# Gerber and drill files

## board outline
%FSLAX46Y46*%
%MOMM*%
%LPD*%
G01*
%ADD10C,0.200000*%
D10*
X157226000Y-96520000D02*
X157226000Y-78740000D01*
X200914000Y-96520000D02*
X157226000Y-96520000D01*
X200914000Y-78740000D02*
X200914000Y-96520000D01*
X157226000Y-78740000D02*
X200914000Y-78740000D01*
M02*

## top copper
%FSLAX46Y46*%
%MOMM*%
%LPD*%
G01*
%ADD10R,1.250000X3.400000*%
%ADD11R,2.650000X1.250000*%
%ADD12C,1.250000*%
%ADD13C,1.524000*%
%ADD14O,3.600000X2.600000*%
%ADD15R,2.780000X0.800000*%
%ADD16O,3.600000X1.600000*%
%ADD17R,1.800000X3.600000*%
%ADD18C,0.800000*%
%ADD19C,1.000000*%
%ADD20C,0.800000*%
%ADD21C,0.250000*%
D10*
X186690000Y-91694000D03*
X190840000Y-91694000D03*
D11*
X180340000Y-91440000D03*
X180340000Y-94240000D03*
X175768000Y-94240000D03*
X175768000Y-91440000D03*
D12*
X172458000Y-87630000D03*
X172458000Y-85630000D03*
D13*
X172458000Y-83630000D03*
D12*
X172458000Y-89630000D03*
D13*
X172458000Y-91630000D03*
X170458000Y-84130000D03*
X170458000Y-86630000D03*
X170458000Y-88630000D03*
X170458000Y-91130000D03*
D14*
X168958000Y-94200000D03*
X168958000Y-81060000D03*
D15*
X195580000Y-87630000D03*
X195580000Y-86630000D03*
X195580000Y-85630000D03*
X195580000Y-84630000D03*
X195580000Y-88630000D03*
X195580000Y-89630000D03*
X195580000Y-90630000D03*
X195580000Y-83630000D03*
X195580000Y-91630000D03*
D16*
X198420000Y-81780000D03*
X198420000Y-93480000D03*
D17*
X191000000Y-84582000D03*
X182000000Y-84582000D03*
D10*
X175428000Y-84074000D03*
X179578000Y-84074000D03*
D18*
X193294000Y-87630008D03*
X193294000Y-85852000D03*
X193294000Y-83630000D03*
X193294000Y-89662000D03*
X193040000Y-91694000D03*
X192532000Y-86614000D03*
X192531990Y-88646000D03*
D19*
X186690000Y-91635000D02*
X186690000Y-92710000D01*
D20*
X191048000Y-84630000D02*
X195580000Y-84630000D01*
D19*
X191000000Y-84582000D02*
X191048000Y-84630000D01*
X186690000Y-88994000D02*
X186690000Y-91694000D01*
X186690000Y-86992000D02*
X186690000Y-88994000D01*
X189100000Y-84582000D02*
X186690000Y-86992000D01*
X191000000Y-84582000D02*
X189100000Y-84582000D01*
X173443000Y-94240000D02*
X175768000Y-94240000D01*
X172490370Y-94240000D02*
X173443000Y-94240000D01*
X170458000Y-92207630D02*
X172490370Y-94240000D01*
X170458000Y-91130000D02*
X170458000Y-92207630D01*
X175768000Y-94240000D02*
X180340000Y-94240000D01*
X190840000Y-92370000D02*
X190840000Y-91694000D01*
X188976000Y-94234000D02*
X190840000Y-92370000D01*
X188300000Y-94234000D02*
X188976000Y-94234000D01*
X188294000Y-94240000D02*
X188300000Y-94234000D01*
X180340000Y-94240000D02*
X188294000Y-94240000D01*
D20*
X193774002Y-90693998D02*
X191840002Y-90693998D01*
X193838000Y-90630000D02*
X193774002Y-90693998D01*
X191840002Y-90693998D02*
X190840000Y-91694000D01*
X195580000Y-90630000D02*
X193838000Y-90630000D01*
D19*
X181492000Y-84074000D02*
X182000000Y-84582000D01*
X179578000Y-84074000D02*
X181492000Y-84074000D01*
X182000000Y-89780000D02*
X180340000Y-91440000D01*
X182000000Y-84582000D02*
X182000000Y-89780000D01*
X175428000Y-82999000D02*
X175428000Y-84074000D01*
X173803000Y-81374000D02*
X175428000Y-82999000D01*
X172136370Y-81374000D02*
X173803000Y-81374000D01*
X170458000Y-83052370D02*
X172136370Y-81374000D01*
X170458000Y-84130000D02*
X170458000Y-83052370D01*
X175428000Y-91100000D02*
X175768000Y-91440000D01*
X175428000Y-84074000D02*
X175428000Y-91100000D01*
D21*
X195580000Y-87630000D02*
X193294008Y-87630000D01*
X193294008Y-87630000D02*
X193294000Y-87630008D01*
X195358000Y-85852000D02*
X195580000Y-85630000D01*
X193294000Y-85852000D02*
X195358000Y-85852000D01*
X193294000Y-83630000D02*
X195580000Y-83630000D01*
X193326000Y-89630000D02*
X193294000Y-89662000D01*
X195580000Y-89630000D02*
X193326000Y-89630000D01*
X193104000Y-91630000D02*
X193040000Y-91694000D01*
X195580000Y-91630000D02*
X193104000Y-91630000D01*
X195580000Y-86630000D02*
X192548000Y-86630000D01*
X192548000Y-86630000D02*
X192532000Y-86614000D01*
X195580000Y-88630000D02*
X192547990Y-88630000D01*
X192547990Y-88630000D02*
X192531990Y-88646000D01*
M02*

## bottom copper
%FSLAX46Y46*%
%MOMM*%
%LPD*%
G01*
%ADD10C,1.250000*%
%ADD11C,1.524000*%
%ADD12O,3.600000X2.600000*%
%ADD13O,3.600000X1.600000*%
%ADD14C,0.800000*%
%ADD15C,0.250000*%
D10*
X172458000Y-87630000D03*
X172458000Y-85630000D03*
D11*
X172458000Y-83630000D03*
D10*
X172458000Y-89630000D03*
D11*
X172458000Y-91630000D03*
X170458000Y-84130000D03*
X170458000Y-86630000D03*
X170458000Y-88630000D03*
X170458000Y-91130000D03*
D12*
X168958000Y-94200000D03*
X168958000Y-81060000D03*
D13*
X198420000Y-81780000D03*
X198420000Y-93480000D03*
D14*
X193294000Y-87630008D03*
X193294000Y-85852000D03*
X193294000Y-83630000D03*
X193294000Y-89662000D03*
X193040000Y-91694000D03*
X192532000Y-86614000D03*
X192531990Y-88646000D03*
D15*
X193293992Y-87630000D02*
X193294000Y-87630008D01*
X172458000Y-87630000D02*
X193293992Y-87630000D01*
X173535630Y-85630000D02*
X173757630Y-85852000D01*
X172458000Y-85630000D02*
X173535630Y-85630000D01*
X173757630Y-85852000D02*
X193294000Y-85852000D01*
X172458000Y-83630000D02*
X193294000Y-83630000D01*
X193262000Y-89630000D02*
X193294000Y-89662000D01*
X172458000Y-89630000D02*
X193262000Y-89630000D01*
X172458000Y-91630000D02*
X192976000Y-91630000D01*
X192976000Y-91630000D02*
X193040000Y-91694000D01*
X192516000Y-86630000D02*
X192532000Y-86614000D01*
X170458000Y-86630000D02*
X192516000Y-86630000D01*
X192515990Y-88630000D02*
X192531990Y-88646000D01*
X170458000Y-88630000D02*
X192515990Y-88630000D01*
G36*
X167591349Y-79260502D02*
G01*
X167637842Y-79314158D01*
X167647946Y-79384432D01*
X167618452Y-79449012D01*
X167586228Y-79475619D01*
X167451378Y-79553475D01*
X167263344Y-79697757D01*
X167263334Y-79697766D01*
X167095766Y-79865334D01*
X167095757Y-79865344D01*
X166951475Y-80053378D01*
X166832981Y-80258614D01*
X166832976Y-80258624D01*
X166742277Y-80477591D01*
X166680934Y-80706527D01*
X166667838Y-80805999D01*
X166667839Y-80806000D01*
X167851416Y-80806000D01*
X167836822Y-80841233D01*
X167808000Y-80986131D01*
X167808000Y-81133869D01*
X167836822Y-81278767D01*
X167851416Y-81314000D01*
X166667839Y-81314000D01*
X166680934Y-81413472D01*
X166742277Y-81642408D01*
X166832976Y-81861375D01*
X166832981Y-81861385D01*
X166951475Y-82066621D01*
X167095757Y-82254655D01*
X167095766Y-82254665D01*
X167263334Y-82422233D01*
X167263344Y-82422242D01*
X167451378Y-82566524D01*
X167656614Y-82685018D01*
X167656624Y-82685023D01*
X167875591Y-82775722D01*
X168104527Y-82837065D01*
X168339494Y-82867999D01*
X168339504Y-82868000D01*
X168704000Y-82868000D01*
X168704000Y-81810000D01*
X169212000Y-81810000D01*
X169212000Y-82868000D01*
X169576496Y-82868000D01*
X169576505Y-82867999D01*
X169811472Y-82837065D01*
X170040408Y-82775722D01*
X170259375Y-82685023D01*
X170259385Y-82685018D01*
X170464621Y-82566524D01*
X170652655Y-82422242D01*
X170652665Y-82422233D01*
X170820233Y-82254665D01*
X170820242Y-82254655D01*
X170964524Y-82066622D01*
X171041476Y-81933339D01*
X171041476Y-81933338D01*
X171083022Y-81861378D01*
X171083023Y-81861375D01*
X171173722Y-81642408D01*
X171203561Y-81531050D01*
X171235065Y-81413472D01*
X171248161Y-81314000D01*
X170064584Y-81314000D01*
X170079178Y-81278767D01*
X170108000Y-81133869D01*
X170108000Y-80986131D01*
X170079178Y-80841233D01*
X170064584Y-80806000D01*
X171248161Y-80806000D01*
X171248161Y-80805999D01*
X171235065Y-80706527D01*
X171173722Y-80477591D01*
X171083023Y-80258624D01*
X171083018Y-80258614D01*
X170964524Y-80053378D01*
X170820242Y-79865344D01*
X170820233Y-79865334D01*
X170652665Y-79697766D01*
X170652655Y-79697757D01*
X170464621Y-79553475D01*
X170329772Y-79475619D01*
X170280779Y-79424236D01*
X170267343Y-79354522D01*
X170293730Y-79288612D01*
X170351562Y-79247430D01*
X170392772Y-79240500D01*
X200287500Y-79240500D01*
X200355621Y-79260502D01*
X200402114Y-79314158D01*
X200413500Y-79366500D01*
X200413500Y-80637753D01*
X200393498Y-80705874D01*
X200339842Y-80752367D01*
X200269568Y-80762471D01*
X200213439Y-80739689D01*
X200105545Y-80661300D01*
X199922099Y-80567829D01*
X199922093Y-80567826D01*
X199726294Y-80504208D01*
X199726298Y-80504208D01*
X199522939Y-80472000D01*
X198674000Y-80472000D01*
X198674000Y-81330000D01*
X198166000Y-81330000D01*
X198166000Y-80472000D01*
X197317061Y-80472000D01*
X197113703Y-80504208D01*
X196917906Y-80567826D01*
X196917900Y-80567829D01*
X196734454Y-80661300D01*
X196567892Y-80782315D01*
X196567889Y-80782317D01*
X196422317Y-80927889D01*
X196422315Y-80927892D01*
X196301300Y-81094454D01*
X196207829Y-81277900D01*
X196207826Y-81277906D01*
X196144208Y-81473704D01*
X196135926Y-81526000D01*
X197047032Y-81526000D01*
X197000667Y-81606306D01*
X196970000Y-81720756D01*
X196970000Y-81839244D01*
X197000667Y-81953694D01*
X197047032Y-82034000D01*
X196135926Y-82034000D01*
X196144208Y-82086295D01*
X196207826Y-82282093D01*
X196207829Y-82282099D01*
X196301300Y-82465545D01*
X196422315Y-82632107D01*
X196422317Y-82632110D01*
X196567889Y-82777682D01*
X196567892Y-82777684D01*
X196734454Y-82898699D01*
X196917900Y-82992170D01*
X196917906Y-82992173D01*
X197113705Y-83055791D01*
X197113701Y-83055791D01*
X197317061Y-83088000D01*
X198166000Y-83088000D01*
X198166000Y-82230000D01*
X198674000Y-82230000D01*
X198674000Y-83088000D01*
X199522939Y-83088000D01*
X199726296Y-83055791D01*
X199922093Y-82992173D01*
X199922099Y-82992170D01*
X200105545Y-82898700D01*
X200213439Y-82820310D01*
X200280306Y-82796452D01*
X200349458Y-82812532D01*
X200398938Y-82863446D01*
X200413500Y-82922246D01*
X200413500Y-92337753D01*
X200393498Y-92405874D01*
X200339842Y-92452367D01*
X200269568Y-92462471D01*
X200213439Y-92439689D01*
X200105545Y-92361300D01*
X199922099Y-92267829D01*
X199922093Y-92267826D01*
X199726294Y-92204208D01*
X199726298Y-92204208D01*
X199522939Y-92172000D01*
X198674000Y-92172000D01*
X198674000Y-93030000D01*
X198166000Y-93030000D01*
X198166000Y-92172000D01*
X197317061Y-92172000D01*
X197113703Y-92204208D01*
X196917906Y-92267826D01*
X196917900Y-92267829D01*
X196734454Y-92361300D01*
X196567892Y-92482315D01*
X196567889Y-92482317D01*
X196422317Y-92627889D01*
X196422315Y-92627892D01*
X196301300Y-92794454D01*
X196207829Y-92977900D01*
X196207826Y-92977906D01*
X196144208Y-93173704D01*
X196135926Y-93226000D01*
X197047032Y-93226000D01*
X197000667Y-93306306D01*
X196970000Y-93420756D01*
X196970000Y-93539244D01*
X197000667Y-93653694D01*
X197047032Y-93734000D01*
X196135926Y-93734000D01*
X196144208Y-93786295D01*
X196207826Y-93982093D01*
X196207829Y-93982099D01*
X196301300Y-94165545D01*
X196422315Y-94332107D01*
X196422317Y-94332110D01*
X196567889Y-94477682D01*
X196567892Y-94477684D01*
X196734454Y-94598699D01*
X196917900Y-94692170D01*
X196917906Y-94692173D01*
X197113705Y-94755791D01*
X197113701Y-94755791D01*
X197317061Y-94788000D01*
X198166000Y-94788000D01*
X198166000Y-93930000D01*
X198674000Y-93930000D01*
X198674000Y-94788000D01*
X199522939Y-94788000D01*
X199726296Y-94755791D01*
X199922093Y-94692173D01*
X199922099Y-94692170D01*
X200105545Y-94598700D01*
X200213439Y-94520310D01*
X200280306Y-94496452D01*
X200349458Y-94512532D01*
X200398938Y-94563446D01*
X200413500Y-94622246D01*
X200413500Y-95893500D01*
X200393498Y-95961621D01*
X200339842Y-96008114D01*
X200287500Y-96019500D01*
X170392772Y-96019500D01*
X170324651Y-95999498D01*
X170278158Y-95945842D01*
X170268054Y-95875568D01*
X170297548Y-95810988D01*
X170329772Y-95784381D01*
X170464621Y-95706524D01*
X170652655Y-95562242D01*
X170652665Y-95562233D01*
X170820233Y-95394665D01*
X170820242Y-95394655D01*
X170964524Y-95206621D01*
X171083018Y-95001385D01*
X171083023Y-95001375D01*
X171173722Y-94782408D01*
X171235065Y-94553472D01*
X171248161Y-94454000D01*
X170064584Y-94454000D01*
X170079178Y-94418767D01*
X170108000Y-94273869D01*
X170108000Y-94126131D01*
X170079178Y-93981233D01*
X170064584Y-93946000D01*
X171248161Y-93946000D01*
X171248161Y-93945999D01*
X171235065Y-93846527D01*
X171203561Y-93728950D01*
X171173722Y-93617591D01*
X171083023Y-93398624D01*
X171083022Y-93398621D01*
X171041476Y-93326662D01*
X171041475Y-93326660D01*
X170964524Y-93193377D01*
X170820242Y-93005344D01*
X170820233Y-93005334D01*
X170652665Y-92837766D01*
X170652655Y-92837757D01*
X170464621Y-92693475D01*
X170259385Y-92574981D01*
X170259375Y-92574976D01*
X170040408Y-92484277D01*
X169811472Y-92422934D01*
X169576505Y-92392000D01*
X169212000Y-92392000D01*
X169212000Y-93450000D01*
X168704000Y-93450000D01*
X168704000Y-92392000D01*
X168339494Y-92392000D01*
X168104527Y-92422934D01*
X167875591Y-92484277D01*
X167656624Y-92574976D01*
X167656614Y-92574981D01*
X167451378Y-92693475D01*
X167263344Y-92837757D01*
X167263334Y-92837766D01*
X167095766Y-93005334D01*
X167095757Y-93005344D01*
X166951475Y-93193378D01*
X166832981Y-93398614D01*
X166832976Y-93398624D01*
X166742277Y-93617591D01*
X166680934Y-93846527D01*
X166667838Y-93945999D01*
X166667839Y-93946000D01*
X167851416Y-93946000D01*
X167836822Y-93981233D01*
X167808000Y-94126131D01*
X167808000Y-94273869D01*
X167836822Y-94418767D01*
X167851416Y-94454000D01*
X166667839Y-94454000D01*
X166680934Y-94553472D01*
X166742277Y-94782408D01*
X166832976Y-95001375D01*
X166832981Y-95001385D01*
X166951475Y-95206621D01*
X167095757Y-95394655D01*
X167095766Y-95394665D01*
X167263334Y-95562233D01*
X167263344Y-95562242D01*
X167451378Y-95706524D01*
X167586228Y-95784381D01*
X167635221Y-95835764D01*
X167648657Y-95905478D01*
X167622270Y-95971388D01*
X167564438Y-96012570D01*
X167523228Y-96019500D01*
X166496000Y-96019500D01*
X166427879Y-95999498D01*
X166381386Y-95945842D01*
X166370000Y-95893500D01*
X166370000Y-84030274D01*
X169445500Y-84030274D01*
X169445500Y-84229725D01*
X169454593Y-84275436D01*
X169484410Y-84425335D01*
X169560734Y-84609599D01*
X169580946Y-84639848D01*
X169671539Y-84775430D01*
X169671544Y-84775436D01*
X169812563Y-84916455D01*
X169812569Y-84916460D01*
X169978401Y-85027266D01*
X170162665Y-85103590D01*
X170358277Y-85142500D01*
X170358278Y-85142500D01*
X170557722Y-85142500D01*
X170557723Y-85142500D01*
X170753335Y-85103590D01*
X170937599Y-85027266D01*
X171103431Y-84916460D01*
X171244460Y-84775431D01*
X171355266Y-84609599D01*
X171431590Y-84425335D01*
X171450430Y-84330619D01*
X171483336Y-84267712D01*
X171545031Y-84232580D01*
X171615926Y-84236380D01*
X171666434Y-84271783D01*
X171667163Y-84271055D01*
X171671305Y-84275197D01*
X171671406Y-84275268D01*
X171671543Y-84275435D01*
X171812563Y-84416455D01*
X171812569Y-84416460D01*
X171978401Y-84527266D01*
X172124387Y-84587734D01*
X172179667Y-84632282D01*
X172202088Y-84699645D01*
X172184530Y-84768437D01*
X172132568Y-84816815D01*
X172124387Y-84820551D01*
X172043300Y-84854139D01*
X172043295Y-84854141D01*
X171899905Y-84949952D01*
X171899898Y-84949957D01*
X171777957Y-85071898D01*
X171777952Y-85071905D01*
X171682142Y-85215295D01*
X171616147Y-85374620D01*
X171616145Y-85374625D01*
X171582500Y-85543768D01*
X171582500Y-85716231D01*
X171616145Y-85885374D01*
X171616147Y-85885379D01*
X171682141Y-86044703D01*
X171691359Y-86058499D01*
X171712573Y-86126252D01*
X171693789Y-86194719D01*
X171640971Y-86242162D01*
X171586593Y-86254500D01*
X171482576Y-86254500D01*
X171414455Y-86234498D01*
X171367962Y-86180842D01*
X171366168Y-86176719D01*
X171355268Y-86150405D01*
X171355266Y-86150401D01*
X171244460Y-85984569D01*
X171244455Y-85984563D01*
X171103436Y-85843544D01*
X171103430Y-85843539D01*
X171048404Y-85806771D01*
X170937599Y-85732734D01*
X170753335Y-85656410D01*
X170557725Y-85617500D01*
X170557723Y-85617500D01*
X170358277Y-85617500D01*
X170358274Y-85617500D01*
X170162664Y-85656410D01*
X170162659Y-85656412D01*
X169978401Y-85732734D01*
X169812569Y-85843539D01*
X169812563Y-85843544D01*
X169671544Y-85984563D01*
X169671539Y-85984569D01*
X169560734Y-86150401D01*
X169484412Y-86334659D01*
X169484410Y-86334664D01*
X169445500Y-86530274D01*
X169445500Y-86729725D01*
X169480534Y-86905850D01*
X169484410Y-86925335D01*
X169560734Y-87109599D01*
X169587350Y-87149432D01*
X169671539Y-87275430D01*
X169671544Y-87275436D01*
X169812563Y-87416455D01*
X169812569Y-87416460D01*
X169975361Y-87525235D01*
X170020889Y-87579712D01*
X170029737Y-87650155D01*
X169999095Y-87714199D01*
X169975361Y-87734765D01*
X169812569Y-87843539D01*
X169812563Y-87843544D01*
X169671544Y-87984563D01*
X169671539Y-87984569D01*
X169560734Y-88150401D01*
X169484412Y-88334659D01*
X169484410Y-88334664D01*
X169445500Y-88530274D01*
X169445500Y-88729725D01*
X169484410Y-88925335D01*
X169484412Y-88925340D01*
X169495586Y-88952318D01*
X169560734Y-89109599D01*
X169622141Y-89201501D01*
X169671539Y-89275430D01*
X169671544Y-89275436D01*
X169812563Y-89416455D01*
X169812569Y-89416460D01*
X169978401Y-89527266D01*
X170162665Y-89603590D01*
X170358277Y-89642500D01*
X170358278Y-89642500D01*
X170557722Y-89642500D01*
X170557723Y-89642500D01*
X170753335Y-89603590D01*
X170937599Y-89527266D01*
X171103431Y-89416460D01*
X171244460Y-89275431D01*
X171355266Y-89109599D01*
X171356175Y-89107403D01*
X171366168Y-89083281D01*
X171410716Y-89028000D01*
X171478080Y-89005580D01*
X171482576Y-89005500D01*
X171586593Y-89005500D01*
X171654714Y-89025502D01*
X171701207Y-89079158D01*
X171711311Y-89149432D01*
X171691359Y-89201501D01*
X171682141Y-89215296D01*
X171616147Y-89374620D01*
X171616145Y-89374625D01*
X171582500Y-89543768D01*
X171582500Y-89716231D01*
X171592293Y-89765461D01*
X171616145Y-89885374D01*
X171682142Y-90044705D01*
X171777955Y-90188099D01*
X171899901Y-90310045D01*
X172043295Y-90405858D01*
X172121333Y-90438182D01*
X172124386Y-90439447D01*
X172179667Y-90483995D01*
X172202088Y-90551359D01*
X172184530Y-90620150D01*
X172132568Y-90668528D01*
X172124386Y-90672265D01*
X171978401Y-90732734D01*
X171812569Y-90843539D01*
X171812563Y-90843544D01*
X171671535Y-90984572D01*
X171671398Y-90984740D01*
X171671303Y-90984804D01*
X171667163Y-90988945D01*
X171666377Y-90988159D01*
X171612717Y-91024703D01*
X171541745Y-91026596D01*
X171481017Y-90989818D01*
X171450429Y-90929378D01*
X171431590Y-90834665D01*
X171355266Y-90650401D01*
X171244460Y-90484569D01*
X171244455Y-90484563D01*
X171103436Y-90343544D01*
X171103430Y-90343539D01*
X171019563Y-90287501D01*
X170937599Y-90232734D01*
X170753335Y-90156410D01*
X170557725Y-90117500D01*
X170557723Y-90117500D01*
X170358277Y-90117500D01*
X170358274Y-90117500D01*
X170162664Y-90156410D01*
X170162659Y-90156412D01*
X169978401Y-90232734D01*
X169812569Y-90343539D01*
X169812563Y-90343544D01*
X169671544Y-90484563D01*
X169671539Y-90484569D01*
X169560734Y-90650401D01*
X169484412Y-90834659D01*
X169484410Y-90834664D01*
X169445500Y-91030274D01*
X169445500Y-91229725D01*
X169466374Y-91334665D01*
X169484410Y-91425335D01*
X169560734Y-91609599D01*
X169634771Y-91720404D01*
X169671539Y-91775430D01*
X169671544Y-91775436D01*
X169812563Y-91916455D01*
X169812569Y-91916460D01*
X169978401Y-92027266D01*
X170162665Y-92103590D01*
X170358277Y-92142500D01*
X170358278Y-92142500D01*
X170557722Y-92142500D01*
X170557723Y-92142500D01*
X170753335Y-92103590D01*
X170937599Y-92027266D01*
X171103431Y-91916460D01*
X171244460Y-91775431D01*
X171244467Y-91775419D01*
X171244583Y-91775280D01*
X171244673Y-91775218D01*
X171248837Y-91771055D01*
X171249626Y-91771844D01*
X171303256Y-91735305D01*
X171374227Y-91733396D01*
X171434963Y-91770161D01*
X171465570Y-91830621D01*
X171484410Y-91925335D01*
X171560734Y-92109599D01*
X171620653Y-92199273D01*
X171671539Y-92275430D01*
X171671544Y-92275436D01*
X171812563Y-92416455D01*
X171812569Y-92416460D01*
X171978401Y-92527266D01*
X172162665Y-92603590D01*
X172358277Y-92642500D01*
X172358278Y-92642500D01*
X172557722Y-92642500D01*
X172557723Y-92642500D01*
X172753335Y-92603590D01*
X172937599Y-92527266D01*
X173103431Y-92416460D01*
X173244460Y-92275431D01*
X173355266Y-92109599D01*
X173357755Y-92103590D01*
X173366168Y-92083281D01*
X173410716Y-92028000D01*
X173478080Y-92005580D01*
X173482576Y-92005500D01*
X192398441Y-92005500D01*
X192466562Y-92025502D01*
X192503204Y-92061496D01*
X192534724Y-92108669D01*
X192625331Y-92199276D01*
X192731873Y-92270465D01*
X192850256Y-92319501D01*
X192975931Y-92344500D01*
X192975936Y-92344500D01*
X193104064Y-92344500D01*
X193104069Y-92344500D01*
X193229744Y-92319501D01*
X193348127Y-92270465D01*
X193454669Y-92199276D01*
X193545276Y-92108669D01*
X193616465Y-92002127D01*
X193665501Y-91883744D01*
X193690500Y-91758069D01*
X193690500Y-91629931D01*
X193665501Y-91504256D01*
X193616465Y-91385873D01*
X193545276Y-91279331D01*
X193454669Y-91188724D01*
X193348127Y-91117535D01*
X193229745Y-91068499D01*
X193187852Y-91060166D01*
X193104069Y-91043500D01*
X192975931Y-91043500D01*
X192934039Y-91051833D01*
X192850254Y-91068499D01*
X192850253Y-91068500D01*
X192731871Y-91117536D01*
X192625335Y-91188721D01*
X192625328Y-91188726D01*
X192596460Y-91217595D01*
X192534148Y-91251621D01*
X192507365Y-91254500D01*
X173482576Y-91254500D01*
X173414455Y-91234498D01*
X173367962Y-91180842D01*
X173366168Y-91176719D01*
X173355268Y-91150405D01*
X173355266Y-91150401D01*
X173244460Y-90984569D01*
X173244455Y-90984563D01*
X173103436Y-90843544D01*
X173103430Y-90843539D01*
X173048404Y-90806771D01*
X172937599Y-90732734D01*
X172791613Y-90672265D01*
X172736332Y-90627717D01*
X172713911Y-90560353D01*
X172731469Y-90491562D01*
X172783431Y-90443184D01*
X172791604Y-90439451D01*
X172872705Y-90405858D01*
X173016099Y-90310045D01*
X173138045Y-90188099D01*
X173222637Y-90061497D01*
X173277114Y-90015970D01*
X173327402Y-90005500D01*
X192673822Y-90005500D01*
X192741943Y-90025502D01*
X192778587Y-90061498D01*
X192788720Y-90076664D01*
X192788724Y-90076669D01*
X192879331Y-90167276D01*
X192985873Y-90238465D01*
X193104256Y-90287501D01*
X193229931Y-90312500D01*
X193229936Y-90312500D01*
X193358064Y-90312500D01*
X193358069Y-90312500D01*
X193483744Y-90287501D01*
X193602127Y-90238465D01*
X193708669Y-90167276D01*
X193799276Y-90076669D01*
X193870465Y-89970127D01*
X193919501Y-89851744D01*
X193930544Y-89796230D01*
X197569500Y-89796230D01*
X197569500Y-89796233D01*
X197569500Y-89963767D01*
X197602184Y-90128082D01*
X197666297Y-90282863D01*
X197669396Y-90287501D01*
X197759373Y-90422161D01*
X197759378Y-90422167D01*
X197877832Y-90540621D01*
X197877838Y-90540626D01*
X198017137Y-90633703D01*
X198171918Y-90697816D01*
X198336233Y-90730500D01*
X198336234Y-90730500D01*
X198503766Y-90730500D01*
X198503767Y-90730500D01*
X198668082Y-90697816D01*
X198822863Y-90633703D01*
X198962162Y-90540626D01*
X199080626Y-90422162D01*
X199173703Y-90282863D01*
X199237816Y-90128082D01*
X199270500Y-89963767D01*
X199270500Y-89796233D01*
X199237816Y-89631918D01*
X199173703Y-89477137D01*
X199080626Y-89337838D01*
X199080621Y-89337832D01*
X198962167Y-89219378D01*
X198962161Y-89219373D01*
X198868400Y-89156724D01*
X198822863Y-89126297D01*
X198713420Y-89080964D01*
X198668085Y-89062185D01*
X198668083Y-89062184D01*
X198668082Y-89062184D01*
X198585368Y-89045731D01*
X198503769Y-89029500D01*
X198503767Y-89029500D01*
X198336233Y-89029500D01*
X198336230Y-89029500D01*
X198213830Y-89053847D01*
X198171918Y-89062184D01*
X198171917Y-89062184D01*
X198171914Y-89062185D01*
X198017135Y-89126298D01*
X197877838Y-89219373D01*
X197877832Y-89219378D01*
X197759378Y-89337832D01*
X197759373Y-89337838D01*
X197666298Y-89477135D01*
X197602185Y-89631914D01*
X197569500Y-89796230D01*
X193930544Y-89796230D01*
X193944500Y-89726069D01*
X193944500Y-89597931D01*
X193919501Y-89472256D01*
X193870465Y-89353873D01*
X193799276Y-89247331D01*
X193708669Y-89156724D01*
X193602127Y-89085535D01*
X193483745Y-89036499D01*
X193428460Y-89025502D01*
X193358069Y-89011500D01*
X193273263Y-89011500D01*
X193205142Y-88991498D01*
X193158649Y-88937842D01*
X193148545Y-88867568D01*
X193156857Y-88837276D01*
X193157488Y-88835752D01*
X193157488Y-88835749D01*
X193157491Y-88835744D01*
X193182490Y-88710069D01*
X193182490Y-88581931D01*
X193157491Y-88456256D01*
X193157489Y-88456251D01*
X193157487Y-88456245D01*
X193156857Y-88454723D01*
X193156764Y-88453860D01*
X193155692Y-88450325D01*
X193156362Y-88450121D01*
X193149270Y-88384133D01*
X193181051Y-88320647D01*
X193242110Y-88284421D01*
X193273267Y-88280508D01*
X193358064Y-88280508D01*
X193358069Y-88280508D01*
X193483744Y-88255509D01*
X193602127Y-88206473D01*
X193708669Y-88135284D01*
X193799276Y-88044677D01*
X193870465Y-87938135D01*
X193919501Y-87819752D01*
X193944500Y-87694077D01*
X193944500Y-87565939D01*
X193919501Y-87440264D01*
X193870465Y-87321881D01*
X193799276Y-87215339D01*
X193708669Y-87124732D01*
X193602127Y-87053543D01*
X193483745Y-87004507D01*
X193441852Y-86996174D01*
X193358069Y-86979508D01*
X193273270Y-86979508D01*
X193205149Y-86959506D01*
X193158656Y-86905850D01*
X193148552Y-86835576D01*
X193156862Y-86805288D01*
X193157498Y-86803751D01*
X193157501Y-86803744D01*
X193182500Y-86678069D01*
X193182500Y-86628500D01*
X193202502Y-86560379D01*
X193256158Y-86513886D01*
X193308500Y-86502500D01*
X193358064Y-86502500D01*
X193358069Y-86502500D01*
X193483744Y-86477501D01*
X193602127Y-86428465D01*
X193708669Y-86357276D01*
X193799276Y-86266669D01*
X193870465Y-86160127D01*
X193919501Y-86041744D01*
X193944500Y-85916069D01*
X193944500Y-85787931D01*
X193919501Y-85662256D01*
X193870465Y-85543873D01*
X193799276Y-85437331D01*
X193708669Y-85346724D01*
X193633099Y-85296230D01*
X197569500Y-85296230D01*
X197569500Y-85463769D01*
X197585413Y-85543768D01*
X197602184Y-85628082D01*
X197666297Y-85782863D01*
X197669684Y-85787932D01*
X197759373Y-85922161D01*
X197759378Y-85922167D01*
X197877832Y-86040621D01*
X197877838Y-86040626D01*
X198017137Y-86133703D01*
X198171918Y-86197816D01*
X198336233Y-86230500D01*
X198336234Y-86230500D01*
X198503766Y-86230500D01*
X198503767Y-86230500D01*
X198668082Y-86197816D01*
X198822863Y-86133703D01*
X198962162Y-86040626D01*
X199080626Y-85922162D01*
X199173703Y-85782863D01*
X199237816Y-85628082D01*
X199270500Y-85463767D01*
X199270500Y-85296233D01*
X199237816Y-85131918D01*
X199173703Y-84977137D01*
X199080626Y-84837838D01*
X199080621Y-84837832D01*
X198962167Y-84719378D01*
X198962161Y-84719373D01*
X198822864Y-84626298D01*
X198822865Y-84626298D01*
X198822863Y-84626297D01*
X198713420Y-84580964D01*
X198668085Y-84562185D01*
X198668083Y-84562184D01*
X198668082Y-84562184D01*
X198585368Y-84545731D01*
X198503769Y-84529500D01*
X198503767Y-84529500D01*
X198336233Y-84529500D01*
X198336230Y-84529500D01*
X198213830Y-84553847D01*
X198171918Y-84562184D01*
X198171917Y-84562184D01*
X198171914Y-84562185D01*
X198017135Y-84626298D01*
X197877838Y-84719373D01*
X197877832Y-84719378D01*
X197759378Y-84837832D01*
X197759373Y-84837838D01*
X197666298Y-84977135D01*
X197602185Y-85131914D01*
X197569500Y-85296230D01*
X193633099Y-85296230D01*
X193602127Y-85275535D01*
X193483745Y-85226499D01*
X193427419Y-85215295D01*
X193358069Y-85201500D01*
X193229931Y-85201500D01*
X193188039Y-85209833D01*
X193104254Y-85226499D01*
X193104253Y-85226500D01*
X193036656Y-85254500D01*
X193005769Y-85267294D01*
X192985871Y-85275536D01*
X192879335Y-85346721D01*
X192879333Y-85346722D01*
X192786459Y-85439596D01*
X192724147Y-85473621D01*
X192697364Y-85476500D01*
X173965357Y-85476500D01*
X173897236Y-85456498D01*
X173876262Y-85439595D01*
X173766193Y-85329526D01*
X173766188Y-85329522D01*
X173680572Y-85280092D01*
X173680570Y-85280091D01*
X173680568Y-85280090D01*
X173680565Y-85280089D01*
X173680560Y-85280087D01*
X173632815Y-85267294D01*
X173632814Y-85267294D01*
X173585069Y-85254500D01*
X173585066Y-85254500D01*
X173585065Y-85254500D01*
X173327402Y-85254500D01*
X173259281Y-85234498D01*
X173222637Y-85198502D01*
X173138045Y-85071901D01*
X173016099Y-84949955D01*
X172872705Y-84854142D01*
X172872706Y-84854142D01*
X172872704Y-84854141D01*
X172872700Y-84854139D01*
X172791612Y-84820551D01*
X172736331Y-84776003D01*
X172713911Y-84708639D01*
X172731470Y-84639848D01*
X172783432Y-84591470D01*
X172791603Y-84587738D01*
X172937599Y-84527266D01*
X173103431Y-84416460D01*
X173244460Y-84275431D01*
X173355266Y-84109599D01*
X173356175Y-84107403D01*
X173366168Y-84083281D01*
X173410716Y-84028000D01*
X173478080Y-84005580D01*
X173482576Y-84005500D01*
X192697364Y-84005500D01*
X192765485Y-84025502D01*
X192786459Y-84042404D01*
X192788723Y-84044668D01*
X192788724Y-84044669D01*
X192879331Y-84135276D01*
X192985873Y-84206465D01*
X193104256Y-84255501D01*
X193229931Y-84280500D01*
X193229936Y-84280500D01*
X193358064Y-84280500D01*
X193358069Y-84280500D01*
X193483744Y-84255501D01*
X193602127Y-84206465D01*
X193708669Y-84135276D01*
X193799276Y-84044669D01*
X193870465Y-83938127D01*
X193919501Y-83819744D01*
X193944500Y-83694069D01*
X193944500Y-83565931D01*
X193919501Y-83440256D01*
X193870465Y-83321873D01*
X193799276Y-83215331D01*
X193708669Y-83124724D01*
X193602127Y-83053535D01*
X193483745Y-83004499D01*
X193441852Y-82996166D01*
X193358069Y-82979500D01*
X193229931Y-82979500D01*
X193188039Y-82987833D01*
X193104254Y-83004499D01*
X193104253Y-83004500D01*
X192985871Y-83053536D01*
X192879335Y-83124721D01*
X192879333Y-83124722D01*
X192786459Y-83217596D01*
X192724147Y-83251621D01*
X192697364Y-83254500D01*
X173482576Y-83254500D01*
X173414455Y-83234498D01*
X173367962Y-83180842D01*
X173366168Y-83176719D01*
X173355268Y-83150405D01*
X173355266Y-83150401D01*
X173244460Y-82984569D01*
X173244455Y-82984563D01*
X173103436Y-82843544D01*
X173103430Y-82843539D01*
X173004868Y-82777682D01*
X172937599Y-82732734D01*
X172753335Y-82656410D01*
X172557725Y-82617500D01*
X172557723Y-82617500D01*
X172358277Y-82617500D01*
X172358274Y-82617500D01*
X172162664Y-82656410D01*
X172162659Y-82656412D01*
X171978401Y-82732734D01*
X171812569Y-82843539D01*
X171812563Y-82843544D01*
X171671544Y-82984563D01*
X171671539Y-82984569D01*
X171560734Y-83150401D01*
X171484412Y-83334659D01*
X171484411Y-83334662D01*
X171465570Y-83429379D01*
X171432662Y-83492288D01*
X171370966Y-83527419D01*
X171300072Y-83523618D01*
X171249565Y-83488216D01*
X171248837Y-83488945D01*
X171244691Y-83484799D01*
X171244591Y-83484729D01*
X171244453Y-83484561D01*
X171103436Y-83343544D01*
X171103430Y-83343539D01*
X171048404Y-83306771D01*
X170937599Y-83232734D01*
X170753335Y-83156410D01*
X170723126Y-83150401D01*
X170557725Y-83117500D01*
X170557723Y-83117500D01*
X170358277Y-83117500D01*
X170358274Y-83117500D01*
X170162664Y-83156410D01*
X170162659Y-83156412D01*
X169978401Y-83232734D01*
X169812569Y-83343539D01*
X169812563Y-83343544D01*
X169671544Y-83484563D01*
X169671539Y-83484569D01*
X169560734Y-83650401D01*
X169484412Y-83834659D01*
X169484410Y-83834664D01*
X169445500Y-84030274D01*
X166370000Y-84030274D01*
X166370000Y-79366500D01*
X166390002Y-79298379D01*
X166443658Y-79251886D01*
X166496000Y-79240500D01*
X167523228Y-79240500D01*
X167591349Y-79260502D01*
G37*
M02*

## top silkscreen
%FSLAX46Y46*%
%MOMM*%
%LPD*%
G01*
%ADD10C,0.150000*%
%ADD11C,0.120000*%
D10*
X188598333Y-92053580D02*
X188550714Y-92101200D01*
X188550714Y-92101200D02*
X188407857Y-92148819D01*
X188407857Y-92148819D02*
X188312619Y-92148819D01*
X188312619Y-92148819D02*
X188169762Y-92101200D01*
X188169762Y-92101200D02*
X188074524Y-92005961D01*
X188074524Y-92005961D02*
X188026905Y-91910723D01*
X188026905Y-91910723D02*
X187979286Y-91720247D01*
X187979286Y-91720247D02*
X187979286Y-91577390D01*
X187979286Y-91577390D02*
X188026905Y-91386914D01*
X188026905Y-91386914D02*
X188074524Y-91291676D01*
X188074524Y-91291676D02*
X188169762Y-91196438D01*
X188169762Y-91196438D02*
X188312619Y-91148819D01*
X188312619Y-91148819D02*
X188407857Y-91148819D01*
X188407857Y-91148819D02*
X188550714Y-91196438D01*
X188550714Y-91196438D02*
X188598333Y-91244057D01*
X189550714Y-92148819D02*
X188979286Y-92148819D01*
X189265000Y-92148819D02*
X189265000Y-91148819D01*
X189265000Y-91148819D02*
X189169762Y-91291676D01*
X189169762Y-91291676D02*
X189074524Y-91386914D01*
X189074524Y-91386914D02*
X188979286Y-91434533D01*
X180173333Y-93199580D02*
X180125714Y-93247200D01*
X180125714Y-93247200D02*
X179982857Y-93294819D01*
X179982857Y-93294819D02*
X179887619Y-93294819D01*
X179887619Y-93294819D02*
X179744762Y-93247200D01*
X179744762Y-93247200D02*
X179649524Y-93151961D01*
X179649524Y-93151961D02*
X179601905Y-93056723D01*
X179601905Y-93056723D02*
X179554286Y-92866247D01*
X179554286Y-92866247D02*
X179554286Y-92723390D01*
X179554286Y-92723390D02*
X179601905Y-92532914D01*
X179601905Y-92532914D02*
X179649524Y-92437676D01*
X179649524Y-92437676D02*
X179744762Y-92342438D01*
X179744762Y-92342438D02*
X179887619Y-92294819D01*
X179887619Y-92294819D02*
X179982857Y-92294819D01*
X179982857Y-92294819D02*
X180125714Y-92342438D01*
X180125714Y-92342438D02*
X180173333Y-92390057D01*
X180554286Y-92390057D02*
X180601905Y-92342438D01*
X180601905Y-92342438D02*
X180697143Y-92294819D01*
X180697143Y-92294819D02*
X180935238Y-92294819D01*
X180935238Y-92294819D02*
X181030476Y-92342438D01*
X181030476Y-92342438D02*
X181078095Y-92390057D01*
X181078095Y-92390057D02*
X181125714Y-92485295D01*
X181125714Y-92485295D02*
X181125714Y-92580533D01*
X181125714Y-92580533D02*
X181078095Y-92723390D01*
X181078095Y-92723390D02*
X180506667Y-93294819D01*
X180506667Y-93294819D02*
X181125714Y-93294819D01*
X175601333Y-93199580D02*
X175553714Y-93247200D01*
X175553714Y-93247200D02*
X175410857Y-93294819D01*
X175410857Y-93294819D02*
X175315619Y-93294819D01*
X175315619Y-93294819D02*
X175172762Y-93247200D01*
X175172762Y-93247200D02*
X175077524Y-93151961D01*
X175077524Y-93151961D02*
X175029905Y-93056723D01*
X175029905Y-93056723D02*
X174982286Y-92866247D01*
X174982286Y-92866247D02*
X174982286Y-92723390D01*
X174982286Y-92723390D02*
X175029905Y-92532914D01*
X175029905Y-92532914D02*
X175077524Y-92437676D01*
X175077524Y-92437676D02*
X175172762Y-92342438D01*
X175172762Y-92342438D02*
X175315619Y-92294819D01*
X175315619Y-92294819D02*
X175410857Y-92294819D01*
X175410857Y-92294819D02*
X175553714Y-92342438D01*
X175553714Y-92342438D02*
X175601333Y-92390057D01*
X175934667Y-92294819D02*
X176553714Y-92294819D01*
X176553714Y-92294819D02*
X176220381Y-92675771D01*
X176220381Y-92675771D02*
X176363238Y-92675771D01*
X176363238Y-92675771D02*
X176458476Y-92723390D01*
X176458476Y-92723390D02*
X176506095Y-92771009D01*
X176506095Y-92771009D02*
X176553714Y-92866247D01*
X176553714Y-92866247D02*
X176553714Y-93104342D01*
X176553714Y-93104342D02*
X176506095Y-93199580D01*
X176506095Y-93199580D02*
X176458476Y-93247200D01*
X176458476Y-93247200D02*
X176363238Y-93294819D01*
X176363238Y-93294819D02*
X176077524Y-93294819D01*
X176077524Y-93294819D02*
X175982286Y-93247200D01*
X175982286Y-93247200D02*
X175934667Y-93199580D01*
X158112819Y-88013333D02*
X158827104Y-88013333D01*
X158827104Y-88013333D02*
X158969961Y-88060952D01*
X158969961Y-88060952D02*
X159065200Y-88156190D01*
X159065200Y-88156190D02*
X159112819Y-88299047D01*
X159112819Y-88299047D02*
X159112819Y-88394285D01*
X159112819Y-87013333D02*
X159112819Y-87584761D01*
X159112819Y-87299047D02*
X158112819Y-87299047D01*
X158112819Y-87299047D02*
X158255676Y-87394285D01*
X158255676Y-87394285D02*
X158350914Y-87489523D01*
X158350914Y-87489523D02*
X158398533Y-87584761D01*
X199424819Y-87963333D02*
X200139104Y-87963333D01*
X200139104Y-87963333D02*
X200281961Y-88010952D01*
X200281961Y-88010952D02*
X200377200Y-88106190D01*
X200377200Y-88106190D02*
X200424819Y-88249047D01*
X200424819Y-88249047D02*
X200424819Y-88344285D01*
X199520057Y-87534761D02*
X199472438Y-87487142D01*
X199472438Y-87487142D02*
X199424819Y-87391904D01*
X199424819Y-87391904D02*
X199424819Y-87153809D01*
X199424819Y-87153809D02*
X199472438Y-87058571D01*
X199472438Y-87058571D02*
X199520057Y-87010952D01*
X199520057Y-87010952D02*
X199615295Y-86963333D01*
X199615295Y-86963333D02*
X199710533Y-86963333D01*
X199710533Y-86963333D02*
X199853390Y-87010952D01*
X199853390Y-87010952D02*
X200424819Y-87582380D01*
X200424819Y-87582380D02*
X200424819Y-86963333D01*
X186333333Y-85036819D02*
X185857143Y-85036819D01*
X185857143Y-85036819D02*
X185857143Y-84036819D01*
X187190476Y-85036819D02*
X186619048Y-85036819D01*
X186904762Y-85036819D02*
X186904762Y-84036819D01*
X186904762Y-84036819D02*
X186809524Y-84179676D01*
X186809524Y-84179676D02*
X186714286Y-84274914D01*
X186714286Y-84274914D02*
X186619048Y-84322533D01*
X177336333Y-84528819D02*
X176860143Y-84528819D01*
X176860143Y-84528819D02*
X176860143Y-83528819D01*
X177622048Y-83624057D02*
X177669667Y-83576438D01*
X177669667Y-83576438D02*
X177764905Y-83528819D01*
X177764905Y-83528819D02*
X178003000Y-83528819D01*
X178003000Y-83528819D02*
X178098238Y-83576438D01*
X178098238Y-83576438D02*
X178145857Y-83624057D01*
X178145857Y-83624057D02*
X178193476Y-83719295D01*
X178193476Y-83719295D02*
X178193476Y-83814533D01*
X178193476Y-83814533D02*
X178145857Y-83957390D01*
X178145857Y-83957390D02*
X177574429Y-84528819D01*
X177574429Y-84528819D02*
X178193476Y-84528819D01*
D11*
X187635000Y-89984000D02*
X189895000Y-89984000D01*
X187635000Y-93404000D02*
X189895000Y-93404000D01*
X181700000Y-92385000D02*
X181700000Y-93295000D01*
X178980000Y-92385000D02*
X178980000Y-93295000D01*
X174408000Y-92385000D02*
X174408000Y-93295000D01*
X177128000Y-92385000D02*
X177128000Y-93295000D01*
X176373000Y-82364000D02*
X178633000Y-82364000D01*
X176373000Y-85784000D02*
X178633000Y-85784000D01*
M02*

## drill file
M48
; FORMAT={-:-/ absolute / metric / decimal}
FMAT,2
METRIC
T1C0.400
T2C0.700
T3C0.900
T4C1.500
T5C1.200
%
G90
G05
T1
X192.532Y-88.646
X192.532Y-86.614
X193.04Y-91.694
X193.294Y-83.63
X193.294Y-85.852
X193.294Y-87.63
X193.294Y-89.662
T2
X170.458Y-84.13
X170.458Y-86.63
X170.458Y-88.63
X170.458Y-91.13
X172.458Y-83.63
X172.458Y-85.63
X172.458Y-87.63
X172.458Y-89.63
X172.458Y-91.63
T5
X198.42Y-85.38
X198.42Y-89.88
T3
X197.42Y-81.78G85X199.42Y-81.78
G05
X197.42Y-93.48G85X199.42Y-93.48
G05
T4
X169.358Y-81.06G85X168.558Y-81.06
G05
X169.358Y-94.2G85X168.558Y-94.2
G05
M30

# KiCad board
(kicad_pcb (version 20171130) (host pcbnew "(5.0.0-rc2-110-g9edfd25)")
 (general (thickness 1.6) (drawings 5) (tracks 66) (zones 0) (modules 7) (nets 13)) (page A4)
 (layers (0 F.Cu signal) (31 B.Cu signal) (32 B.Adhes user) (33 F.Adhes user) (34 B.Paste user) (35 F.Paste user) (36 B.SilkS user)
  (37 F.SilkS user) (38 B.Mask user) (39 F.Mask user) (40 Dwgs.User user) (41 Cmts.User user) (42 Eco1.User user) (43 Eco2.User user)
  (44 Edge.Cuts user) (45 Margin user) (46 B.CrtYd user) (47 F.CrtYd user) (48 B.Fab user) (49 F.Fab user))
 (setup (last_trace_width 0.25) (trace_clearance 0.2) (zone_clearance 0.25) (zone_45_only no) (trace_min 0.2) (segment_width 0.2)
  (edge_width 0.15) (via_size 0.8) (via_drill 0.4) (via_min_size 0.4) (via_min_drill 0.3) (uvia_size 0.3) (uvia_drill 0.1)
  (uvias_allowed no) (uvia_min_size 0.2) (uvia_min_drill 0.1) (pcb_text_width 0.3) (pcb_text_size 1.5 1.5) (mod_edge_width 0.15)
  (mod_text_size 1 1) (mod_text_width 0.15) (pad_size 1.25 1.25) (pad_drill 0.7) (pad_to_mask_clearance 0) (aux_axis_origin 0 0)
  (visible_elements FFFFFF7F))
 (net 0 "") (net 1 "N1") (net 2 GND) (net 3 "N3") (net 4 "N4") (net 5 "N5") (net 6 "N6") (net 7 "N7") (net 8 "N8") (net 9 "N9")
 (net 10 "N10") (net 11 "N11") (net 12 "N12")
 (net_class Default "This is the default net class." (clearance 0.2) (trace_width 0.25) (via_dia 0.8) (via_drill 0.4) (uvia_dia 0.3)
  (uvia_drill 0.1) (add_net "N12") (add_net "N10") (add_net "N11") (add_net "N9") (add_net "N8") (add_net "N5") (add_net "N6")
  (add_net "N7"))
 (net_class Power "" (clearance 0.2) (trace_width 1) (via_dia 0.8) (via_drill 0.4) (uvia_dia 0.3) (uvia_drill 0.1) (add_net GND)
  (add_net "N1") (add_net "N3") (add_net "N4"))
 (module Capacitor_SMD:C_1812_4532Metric (layer F.Cu) (at 188.765 91.694)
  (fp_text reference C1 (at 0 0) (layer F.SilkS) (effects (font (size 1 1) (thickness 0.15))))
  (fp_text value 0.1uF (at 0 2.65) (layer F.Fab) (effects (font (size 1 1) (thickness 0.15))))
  (fp_line (start -1.13 -1.71) (end 1.13 -1.71) (layer F.SilkS) (width 0.12))
  (fp_line (start -1.13 1.71) (end 1.13 1.71) (layer F.SilkS) (width 0.12))
  (pad 1 smd rect (at -2.075 0) (size 1.25 3.4) (layers F.Cu F.Paste F.Mask) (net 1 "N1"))
  (pad 2 smd rect (at 2.075 0) (size 1.25 3.4) (layers F.Cu F.Paste F.Mask) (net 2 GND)))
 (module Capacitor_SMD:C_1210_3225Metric (layer F.Cu) (at 180.34 92.84 270)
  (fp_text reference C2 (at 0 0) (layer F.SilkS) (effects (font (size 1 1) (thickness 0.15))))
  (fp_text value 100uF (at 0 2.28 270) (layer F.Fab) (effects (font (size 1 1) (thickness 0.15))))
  (fp_line (start -0.455 -1.36) (end 0.455 -1.36) (layer F.SilkS) (width 0.12))
  (fp_line (start -0.455 1.36) (end 0.455 1.36) (layer F.SilkS) (width 0.12))
  (pad 1 smd rect (at -1.4 0 270) (size 1.25 2.65) (layers F.Cu F.Paste F.Mask) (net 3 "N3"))
  (pad 2 smd rect (at 1.4 0 270) (size 1.25 2.65) (layers F.Cu F.Paste F.Mask) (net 2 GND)))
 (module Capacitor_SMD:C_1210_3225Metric (layer F.Cu) (at 175.768 92.84 270)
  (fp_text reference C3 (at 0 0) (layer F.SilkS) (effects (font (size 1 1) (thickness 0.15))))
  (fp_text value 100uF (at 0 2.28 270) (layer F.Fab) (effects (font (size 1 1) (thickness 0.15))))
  (fp_line (start -0.455 1.36) (end 0.455 1.36) (layer F.SilkS) (width 0.12))
  (fp_line (start -0.455 -1.36) (end 0.455 -1.36) (layer F.SilkS) (width 0.12))
  (pad 2 smd rect (at 1.4 0 270) (size 1.25 2.65) (layers F.Cu F.Paste F.Mask) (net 2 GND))
  (pad 1 smd rect (at -1.4 0 270) (size 1.25 2.65) (layers F.Cu F.Paste F.Mask) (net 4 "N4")))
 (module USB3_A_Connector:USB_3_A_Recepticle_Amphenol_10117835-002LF (layer F.Cu) (at 165.608 87.63 270)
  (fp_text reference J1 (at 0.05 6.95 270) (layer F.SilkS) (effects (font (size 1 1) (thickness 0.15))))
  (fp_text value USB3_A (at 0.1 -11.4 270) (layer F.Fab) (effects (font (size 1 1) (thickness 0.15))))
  (pad 7 thru_hole circle (at 0 -6.85 270) (size 1.25 1.25) (drill 0.7) (layers *.Cu *.Mask) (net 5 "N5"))
  (pad 8 thru_hole circle (at -2 -6.85 270) (size 1.25 1.25) (drill 0.7) (layers *.Cu *.Mask) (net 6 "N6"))
  (pad 9 thru_hole circle (at -4 -6.85 270) (size 1.524 1.524) (drill 0.7) (layers *.Cu *.Mask) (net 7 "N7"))
  (pad 6 thru_hole circle (at 2 -6.85 270) (size 1.25 1.25) (drill 0.7) (layers *.Cu *.Mask) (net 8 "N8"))
  (pad 5 thru_hole circle (at 4 -6.85 270) (size 1.524 1.524) (drill 0.7) (layers *.Cu *.Mask) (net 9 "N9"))
  (pad 1 thru_hole circle (at -3.5 -4.85 270) (size 1.524 1.524) (drill 0.7) (layers *.Cu *.Mask) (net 4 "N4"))
  (pad 2 thru_hole circle (at -1 -4.85 270) (size 1.524 1.524) (drill 0.7) (layers *.Cu *.Mask) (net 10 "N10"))
  (pad 3 thru_hole circle (at 1 -4.85 270) (size 1.524 1.524) (drill 0.7) (layers *.Cu *.Mask) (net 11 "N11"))
  (pad 4 thru_hole circle (at 3.5 -4.85 270) (size 1.524 1.524) (drill 0.7) (layers *.Cu *.Mask) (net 2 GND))
  (pad 10 thru_hole oval (at 6.57 -3.35 270) (size 2.6 3.6) (drill oval 1.5 2.3) (layers *.Cu *.Mask) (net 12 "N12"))
  (pad 10 thru_hole oval (at -6.57 -3.35 270) (size 2.6 3.6) (drill oval 1.5 2.3) (layers *.Cu *.Mask) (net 12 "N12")))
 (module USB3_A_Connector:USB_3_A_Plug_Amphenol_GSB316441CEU (layer F.Cu) (at 200.97 87.63 90)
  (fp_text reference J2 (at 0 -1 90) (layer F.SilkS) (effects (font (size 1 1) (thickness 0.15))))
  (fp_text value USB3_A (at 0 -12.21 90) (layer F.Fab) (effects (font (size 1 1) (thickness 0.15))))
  (pad 7 smd rect (at 0 -5.39 90) (size 0.8 2.78) (layers F.Cu F.Paste F.Mask) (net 5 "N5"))
  (pad 2 smd rect (at 1 -5.39 90) (size 0.8 2.78) (layers F.Cu F.Paste F.Mask) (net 10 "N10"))
  (pad 8 smd rect (at 2 -5.39 90) (size 0.8 2.78) (layers F.Cu F.Paste F.Mask) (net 6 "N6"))
  (pad 1 smd rect (at 3 -5.39 90) (size 0.8 2.78) (layers F.Cu F.Paste F.Mask) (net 1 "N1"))
  (pad 3 smd rect (at -1 -5.39 90) (size 0.8 2.78) (layers F.Cu F.Paste F.Mask) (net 11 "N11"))
  (pad 6 smd rect (at -2 -5.39 90) (size 0.8 2.78) (layers F.Cu F.Paste F.Mask) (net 8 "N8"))
  (pad 4 smd rect (at -3 -5.39 90) (size 0.8 2.78) (layers F.Cu F.Paste F.Mask) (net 2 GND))
  (pad 9 smd rect (at 4 -5.39 90) (size 0.8 2.78) (layers F.Cu F.Paste F.Mask) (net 7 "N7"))
  (pad 5 smd rect (at -4 -5.39 90) (size 0.8 2.78) (layers F.Cu F.Paste F.Mask) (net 9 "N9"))
  (pad 10 thru_hole oval (at 5.85 -2.55 90) (size 1.6 3.6) (drill oval 0.9 2.9) (layers *.Cu *.Mask) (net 12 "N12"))
  (pad 10 thru_hole oval (at -5.85 -2.55 90) (size 1.6 3.6) (drill oval 0.9 2.9) (layers *.Cu *.Mask) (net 12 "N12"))
  (pad "" np_thru_hole circle (at 2.25 -2.55 90) (size 1.2 1.2) (drill 1.2) (layers *.Cu *.Mask))
  (pad "" np_thru_hole circle (at -2.25 -2.55 90) (size 1.2 1.2) (drill 1.2) (layers *.Cu *.Mask)))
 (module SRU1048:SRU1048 (layer F.Cu) (at 186.5 84.582)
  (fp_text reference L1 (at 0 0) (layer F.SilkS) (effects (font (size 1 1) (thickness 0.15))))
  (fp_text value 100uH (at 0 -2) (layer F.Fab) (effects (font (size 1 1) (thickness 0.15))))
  (pad 1 smd rect (at 4.5 0) (size 1.8 3.6) (layers F.Cu F.Paste F.Mask) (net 1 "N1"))
  (pad 2 smd rect (at -4.5 0) (size 1.8 3.6) (layers F.Cu F.Paste F.Mask) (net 3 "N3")))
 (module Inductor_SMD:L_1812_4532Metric (layer F.Cu) (at 177.503 84.074)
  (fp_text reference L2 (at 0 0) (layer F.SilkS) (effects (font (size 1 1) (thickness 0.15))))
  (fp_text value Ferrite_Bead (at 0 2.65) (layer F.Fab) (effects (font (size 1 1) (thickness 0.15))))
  (fp_line (start -1.13 -1.71) (end 1.13 -1.71) (layer F.SilkS) (width 0.12))
  (fp_line (start -1.13 1.71) (end 1.13 1.71) (layer F.SilkS) (width 0.12))
  (pad 1 smd rect (at -2.075 0) (size 1.25 3.4) (layers F.Cu F.Paste F.Mask) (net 4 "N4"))
  (pad 2 smd rect (at 2.075 0) (size 1.25 3.4) (layers F.Cu F.Paste F.Mask) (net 3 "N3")))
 (gr_line (start 157.226 96.52) (end 157.226 78.74) (layer Edge.Cuts) (width 0.2))
 (gr_line (start 200.914 96.52) (end 157.226 96.52) (layer Edge.Cuts) (width 0.2))
 (gr_line (start 200.914 78.74) (end 200.914 96.52) (layer Edge.Cuts) (width 0.2))
 (gr_line (start 157.226 78.74) (end 200.914 78.74) (layer Edge.Cuts) (width 0.2))
 (segment (start 186.69 91.635) (end 186.69 92.71) (width 1) (layer F.Cu) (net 1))
 (segment (start 191.048 84.63) (end 195.58 84.63) (width 0.8) (layer F.Cu) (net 1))
 (segment (start 191 84.582) (end 191.048 84.63) (width 1) (layer F.Cu) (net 1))
 (segment (start 186.69 88.994) (end 186.69 91.694) (width 1) (layer F.Cu) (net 1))
 (segment (start 186.69 86.992) (end 186.69 88.994) (width 1) (layer F.Cu) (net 1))
 (segment (start 189.1 84.582) (end 186.69 86.992) (width 1) (layer F.Cu) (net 1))
 (segment (start 191 84.582) (end 189.1 84.582) (width 1) (layer F.Cu) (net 1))
 (segment (start 173.443 94.24) (end 175.768 94.24) (width 1) (layer F.Cu) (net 2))
 (segment (start 172.49037 94.24) (end 173.443 94.24) (width 1) (layer F.Cu) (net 2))
 (segment (start 170.458 92.20763) (end 172.49037 94.24) (width 1) (layer F.Cu) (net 2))
 (segment (start 170.458 91.13) (end 170.458 92.20763) (width 1) (layer F.Cu) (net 2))
 (segment (start 175.768 94.24) (end 180.34 94.24) (width 1) (layer F.Cu) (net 2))
 (segment (start 190.84 92.37) (end 190.84 91.694) (width 1) (layer F.Cu) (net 2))
 (segment (start 188.976 94.234) (end 190.84 92.37) (width 1) (layer F.Cu) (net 2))
 (segment (start 188.3 94.234) (end 188.976 94.234) (width 1) (layer F.Cu) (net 2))
 (segment (start 188.294 94.24) (end 188.3 94.234) (width 1) (layer F.Cu) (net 2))
 (segment (start 180.34 94.24) (end 188.294 94.24) (width 1) (layer F.Cu) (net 2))
 (segment (start 193.774002 90.693998) (end 191.840002 90.693998) (width 0.8) (layer F.Cu) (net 2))
 (segment (start 193.838 90.63) (end 193.774002 90.693998) (width 0.8) (layer F.Cu) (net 2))
 (segment (start 191.840002 90.693998) (end 190.84 91.694) (width 0.8) (layer F.Cu) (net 2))
 (segment (start 195.58 90.63) (end 193.838 90.63) (width 0.8) (layer F.Cu) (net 2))
 (segment (start 181.492 84.074) (end 182 84.582) (width 1) (layer F.Cu) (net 3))
 (segment (start 179.578 84.074) (end 181.492 84.074) (width 1) (layer F.Cu) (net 3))
 (segment (start 182 89.78) (end 180.34 91.44) (width 1) (layer F.Cu) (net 3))
 (segment (start 182 84.582) (end 182 89.78) (width 1) (layer F.Cu) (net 3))
 (segment (start 175.428 82.999) (end 175.428 84.074) (width 1) (layer F.Cu) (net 4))
 (segment (start 173.803 81.374) (end 175.428 82.999) (width 1) (layer F.Cu) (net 4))
 (segment (start 172.13637 81.374) (end 173.803 81.374) (width 1) (layer F.Cu) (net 4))
 (segment (start 170.458 83.05237) (end 172.13637 81.374) (width 1) (layer F.Cu) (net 4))
 (segment (start 170.458 84.13) (end 170.458 83.05237) (width 1) (layer F.Cu) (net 4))
 (segment (start 175.428 91.1) (end 175.768 91.44) (width 1) (layer F.Cu) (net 4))
 (segment (start 175.428 84.074) (end 175.428 91.1) (width 1) (layer F.Cu) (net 4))
 (via (at 193.294 87.630008) (size 0.8) (drill 0.4) (layers F.Cu B.Cu) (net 5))
 (segment (start 193.293992 87.63) (end 193.294 87.630008) (width 0.25) (layer B.Cu) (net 5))
 (segment (start 172.458 87.63) (end 193.293992 87.63) (width 0.25) (layer B.Cu) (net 5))
 (segment (start 195.58 87.63) (end 193.294008 87.63) (width 0.25) (layer F.Cu) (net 5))
 (segment (start 193.294008 87.63) (end 193.294 87.630008) (width 0.25) (layer F.Cu) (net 5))
 (segment (start 173.53563 85.63) (end 173.75763 85.852) (width 0.25) (layer B.Cu) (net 6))
 (segment (start 172.458 85.63) (end 173.53563 85.63) (width 0.25) (layer B.Cu) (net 6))
 (via (at 193.294 85.852) (size 0.8) (drill 0.4) (layers F.Cu B.Cu) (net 6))
 (segment (start 173.75763 85.852) (end 193.294 85.852) (width 0.25) (layer B.Cu) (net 6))
 (segment (start 195.358 85.852) (end 195.58 85.63) (width 0.25) (layer F.Cu) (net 6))
 (segment (start 193.294 85.852) (end 195.358 85.852) (width 0.25) (layer F.Cu) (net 6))
 (via (at 193.294 83.63) (size 0.8) (drill 0.4) (layers F.Cu B.Cu) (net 7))
 (segment (start 172.458 83.63) (end 193.294 83.63) (width 0.25) (layer B.Cu) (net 7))
 (segment (start 193.294 83.63) (end 195.58 83.63) (width 0.25) (layer F.Cu) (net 7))
 (segment (start 193.326 89.63) (end 193.294 89.662) (width 0.25) (layer F.Cu) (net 8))
 (segment (start 195.58 89.63) (end 193.326 89.63) (width 0.25) (layer F.Cu) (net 8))
 (segment (start 193.262 89.63) (end 193.294 89.662) (width 0.25) (layer B.Cu) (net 8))
 (segment (start 172.458 89.63) (end 193.262 89.63) (width 0.25) (layer B.Cu) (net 8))
 (via (at 193.294 89.662) (size 0.8) (drill 0.4) (layers F.Cu B.Cu) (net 8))
 (segment (start 172.458 91.63) (end 192.976 91.63) (width 0.25) (layer B.Cu) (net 9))
 (segment (start 193.104 91.63) (end 193.04 91.694) (width 0.25) (layer F.Cu) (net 9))
 (segment (start 195.58 91.63) (end 193.104 91.63) (width 0.25) (layer F.Cu) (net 9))
 (via (at 193.04 91.694) (size 0.8) (drill 0.4) (layers F.Cu B.Cu) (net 9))
 (segment (start 192.976 91.63) (end 193.04 91.694) (width 0.25) (layer B.Cu) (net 9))
 (via (at 192.532 86.614) (size 0.8) (drill 0.4) (layers F.Cu B.Cu) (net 10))
 (segment (start 195.58 86.63) (end 192.548 86.63) (width 0.25) (layer F.Cu) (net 10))
 (segment (start 192.548 86.63) (end 192.532 86.614) (width 0.25) (layer F.Cu) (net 10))
 (segment (start 192.516 86.63) (end 192.532 86.614) (width 0.25) (layer B.Cu) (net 10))
 (segment (start 170.458 86.63) (end 192.516 86.63) (width 0.25) (layer B.Cu) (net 10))
 (via (at 192.53199 88.646) (size 0.8) (drill 0.4) (layers F.Cu B.Cu) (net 11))
 (segment (start 195.58 88.63) (end 192.54799 88.63) (width 0.25) (layer F.Cu) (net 11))
 (segment (start 192.54799 88.63) (end 192.53199 88.646) (width 0.25) (layer F.Cu) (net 11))
 (segment (start 192.51599 88.63) (end 192.53199 88.646) (width 0.25) (layer B.Cu) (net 11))
 (segment (start 170.458 88.63) (end 192.51599 88.63) (width 0.25) (layer B.Cu) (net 11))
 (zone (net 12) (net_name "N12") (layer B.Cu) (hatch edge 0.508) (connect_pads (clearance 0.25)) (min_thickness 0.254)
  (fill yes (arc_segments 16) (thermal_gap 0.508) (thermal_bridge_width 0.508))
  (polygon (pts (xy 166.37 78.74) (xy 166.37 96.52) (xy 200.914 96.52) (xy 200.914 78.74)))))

